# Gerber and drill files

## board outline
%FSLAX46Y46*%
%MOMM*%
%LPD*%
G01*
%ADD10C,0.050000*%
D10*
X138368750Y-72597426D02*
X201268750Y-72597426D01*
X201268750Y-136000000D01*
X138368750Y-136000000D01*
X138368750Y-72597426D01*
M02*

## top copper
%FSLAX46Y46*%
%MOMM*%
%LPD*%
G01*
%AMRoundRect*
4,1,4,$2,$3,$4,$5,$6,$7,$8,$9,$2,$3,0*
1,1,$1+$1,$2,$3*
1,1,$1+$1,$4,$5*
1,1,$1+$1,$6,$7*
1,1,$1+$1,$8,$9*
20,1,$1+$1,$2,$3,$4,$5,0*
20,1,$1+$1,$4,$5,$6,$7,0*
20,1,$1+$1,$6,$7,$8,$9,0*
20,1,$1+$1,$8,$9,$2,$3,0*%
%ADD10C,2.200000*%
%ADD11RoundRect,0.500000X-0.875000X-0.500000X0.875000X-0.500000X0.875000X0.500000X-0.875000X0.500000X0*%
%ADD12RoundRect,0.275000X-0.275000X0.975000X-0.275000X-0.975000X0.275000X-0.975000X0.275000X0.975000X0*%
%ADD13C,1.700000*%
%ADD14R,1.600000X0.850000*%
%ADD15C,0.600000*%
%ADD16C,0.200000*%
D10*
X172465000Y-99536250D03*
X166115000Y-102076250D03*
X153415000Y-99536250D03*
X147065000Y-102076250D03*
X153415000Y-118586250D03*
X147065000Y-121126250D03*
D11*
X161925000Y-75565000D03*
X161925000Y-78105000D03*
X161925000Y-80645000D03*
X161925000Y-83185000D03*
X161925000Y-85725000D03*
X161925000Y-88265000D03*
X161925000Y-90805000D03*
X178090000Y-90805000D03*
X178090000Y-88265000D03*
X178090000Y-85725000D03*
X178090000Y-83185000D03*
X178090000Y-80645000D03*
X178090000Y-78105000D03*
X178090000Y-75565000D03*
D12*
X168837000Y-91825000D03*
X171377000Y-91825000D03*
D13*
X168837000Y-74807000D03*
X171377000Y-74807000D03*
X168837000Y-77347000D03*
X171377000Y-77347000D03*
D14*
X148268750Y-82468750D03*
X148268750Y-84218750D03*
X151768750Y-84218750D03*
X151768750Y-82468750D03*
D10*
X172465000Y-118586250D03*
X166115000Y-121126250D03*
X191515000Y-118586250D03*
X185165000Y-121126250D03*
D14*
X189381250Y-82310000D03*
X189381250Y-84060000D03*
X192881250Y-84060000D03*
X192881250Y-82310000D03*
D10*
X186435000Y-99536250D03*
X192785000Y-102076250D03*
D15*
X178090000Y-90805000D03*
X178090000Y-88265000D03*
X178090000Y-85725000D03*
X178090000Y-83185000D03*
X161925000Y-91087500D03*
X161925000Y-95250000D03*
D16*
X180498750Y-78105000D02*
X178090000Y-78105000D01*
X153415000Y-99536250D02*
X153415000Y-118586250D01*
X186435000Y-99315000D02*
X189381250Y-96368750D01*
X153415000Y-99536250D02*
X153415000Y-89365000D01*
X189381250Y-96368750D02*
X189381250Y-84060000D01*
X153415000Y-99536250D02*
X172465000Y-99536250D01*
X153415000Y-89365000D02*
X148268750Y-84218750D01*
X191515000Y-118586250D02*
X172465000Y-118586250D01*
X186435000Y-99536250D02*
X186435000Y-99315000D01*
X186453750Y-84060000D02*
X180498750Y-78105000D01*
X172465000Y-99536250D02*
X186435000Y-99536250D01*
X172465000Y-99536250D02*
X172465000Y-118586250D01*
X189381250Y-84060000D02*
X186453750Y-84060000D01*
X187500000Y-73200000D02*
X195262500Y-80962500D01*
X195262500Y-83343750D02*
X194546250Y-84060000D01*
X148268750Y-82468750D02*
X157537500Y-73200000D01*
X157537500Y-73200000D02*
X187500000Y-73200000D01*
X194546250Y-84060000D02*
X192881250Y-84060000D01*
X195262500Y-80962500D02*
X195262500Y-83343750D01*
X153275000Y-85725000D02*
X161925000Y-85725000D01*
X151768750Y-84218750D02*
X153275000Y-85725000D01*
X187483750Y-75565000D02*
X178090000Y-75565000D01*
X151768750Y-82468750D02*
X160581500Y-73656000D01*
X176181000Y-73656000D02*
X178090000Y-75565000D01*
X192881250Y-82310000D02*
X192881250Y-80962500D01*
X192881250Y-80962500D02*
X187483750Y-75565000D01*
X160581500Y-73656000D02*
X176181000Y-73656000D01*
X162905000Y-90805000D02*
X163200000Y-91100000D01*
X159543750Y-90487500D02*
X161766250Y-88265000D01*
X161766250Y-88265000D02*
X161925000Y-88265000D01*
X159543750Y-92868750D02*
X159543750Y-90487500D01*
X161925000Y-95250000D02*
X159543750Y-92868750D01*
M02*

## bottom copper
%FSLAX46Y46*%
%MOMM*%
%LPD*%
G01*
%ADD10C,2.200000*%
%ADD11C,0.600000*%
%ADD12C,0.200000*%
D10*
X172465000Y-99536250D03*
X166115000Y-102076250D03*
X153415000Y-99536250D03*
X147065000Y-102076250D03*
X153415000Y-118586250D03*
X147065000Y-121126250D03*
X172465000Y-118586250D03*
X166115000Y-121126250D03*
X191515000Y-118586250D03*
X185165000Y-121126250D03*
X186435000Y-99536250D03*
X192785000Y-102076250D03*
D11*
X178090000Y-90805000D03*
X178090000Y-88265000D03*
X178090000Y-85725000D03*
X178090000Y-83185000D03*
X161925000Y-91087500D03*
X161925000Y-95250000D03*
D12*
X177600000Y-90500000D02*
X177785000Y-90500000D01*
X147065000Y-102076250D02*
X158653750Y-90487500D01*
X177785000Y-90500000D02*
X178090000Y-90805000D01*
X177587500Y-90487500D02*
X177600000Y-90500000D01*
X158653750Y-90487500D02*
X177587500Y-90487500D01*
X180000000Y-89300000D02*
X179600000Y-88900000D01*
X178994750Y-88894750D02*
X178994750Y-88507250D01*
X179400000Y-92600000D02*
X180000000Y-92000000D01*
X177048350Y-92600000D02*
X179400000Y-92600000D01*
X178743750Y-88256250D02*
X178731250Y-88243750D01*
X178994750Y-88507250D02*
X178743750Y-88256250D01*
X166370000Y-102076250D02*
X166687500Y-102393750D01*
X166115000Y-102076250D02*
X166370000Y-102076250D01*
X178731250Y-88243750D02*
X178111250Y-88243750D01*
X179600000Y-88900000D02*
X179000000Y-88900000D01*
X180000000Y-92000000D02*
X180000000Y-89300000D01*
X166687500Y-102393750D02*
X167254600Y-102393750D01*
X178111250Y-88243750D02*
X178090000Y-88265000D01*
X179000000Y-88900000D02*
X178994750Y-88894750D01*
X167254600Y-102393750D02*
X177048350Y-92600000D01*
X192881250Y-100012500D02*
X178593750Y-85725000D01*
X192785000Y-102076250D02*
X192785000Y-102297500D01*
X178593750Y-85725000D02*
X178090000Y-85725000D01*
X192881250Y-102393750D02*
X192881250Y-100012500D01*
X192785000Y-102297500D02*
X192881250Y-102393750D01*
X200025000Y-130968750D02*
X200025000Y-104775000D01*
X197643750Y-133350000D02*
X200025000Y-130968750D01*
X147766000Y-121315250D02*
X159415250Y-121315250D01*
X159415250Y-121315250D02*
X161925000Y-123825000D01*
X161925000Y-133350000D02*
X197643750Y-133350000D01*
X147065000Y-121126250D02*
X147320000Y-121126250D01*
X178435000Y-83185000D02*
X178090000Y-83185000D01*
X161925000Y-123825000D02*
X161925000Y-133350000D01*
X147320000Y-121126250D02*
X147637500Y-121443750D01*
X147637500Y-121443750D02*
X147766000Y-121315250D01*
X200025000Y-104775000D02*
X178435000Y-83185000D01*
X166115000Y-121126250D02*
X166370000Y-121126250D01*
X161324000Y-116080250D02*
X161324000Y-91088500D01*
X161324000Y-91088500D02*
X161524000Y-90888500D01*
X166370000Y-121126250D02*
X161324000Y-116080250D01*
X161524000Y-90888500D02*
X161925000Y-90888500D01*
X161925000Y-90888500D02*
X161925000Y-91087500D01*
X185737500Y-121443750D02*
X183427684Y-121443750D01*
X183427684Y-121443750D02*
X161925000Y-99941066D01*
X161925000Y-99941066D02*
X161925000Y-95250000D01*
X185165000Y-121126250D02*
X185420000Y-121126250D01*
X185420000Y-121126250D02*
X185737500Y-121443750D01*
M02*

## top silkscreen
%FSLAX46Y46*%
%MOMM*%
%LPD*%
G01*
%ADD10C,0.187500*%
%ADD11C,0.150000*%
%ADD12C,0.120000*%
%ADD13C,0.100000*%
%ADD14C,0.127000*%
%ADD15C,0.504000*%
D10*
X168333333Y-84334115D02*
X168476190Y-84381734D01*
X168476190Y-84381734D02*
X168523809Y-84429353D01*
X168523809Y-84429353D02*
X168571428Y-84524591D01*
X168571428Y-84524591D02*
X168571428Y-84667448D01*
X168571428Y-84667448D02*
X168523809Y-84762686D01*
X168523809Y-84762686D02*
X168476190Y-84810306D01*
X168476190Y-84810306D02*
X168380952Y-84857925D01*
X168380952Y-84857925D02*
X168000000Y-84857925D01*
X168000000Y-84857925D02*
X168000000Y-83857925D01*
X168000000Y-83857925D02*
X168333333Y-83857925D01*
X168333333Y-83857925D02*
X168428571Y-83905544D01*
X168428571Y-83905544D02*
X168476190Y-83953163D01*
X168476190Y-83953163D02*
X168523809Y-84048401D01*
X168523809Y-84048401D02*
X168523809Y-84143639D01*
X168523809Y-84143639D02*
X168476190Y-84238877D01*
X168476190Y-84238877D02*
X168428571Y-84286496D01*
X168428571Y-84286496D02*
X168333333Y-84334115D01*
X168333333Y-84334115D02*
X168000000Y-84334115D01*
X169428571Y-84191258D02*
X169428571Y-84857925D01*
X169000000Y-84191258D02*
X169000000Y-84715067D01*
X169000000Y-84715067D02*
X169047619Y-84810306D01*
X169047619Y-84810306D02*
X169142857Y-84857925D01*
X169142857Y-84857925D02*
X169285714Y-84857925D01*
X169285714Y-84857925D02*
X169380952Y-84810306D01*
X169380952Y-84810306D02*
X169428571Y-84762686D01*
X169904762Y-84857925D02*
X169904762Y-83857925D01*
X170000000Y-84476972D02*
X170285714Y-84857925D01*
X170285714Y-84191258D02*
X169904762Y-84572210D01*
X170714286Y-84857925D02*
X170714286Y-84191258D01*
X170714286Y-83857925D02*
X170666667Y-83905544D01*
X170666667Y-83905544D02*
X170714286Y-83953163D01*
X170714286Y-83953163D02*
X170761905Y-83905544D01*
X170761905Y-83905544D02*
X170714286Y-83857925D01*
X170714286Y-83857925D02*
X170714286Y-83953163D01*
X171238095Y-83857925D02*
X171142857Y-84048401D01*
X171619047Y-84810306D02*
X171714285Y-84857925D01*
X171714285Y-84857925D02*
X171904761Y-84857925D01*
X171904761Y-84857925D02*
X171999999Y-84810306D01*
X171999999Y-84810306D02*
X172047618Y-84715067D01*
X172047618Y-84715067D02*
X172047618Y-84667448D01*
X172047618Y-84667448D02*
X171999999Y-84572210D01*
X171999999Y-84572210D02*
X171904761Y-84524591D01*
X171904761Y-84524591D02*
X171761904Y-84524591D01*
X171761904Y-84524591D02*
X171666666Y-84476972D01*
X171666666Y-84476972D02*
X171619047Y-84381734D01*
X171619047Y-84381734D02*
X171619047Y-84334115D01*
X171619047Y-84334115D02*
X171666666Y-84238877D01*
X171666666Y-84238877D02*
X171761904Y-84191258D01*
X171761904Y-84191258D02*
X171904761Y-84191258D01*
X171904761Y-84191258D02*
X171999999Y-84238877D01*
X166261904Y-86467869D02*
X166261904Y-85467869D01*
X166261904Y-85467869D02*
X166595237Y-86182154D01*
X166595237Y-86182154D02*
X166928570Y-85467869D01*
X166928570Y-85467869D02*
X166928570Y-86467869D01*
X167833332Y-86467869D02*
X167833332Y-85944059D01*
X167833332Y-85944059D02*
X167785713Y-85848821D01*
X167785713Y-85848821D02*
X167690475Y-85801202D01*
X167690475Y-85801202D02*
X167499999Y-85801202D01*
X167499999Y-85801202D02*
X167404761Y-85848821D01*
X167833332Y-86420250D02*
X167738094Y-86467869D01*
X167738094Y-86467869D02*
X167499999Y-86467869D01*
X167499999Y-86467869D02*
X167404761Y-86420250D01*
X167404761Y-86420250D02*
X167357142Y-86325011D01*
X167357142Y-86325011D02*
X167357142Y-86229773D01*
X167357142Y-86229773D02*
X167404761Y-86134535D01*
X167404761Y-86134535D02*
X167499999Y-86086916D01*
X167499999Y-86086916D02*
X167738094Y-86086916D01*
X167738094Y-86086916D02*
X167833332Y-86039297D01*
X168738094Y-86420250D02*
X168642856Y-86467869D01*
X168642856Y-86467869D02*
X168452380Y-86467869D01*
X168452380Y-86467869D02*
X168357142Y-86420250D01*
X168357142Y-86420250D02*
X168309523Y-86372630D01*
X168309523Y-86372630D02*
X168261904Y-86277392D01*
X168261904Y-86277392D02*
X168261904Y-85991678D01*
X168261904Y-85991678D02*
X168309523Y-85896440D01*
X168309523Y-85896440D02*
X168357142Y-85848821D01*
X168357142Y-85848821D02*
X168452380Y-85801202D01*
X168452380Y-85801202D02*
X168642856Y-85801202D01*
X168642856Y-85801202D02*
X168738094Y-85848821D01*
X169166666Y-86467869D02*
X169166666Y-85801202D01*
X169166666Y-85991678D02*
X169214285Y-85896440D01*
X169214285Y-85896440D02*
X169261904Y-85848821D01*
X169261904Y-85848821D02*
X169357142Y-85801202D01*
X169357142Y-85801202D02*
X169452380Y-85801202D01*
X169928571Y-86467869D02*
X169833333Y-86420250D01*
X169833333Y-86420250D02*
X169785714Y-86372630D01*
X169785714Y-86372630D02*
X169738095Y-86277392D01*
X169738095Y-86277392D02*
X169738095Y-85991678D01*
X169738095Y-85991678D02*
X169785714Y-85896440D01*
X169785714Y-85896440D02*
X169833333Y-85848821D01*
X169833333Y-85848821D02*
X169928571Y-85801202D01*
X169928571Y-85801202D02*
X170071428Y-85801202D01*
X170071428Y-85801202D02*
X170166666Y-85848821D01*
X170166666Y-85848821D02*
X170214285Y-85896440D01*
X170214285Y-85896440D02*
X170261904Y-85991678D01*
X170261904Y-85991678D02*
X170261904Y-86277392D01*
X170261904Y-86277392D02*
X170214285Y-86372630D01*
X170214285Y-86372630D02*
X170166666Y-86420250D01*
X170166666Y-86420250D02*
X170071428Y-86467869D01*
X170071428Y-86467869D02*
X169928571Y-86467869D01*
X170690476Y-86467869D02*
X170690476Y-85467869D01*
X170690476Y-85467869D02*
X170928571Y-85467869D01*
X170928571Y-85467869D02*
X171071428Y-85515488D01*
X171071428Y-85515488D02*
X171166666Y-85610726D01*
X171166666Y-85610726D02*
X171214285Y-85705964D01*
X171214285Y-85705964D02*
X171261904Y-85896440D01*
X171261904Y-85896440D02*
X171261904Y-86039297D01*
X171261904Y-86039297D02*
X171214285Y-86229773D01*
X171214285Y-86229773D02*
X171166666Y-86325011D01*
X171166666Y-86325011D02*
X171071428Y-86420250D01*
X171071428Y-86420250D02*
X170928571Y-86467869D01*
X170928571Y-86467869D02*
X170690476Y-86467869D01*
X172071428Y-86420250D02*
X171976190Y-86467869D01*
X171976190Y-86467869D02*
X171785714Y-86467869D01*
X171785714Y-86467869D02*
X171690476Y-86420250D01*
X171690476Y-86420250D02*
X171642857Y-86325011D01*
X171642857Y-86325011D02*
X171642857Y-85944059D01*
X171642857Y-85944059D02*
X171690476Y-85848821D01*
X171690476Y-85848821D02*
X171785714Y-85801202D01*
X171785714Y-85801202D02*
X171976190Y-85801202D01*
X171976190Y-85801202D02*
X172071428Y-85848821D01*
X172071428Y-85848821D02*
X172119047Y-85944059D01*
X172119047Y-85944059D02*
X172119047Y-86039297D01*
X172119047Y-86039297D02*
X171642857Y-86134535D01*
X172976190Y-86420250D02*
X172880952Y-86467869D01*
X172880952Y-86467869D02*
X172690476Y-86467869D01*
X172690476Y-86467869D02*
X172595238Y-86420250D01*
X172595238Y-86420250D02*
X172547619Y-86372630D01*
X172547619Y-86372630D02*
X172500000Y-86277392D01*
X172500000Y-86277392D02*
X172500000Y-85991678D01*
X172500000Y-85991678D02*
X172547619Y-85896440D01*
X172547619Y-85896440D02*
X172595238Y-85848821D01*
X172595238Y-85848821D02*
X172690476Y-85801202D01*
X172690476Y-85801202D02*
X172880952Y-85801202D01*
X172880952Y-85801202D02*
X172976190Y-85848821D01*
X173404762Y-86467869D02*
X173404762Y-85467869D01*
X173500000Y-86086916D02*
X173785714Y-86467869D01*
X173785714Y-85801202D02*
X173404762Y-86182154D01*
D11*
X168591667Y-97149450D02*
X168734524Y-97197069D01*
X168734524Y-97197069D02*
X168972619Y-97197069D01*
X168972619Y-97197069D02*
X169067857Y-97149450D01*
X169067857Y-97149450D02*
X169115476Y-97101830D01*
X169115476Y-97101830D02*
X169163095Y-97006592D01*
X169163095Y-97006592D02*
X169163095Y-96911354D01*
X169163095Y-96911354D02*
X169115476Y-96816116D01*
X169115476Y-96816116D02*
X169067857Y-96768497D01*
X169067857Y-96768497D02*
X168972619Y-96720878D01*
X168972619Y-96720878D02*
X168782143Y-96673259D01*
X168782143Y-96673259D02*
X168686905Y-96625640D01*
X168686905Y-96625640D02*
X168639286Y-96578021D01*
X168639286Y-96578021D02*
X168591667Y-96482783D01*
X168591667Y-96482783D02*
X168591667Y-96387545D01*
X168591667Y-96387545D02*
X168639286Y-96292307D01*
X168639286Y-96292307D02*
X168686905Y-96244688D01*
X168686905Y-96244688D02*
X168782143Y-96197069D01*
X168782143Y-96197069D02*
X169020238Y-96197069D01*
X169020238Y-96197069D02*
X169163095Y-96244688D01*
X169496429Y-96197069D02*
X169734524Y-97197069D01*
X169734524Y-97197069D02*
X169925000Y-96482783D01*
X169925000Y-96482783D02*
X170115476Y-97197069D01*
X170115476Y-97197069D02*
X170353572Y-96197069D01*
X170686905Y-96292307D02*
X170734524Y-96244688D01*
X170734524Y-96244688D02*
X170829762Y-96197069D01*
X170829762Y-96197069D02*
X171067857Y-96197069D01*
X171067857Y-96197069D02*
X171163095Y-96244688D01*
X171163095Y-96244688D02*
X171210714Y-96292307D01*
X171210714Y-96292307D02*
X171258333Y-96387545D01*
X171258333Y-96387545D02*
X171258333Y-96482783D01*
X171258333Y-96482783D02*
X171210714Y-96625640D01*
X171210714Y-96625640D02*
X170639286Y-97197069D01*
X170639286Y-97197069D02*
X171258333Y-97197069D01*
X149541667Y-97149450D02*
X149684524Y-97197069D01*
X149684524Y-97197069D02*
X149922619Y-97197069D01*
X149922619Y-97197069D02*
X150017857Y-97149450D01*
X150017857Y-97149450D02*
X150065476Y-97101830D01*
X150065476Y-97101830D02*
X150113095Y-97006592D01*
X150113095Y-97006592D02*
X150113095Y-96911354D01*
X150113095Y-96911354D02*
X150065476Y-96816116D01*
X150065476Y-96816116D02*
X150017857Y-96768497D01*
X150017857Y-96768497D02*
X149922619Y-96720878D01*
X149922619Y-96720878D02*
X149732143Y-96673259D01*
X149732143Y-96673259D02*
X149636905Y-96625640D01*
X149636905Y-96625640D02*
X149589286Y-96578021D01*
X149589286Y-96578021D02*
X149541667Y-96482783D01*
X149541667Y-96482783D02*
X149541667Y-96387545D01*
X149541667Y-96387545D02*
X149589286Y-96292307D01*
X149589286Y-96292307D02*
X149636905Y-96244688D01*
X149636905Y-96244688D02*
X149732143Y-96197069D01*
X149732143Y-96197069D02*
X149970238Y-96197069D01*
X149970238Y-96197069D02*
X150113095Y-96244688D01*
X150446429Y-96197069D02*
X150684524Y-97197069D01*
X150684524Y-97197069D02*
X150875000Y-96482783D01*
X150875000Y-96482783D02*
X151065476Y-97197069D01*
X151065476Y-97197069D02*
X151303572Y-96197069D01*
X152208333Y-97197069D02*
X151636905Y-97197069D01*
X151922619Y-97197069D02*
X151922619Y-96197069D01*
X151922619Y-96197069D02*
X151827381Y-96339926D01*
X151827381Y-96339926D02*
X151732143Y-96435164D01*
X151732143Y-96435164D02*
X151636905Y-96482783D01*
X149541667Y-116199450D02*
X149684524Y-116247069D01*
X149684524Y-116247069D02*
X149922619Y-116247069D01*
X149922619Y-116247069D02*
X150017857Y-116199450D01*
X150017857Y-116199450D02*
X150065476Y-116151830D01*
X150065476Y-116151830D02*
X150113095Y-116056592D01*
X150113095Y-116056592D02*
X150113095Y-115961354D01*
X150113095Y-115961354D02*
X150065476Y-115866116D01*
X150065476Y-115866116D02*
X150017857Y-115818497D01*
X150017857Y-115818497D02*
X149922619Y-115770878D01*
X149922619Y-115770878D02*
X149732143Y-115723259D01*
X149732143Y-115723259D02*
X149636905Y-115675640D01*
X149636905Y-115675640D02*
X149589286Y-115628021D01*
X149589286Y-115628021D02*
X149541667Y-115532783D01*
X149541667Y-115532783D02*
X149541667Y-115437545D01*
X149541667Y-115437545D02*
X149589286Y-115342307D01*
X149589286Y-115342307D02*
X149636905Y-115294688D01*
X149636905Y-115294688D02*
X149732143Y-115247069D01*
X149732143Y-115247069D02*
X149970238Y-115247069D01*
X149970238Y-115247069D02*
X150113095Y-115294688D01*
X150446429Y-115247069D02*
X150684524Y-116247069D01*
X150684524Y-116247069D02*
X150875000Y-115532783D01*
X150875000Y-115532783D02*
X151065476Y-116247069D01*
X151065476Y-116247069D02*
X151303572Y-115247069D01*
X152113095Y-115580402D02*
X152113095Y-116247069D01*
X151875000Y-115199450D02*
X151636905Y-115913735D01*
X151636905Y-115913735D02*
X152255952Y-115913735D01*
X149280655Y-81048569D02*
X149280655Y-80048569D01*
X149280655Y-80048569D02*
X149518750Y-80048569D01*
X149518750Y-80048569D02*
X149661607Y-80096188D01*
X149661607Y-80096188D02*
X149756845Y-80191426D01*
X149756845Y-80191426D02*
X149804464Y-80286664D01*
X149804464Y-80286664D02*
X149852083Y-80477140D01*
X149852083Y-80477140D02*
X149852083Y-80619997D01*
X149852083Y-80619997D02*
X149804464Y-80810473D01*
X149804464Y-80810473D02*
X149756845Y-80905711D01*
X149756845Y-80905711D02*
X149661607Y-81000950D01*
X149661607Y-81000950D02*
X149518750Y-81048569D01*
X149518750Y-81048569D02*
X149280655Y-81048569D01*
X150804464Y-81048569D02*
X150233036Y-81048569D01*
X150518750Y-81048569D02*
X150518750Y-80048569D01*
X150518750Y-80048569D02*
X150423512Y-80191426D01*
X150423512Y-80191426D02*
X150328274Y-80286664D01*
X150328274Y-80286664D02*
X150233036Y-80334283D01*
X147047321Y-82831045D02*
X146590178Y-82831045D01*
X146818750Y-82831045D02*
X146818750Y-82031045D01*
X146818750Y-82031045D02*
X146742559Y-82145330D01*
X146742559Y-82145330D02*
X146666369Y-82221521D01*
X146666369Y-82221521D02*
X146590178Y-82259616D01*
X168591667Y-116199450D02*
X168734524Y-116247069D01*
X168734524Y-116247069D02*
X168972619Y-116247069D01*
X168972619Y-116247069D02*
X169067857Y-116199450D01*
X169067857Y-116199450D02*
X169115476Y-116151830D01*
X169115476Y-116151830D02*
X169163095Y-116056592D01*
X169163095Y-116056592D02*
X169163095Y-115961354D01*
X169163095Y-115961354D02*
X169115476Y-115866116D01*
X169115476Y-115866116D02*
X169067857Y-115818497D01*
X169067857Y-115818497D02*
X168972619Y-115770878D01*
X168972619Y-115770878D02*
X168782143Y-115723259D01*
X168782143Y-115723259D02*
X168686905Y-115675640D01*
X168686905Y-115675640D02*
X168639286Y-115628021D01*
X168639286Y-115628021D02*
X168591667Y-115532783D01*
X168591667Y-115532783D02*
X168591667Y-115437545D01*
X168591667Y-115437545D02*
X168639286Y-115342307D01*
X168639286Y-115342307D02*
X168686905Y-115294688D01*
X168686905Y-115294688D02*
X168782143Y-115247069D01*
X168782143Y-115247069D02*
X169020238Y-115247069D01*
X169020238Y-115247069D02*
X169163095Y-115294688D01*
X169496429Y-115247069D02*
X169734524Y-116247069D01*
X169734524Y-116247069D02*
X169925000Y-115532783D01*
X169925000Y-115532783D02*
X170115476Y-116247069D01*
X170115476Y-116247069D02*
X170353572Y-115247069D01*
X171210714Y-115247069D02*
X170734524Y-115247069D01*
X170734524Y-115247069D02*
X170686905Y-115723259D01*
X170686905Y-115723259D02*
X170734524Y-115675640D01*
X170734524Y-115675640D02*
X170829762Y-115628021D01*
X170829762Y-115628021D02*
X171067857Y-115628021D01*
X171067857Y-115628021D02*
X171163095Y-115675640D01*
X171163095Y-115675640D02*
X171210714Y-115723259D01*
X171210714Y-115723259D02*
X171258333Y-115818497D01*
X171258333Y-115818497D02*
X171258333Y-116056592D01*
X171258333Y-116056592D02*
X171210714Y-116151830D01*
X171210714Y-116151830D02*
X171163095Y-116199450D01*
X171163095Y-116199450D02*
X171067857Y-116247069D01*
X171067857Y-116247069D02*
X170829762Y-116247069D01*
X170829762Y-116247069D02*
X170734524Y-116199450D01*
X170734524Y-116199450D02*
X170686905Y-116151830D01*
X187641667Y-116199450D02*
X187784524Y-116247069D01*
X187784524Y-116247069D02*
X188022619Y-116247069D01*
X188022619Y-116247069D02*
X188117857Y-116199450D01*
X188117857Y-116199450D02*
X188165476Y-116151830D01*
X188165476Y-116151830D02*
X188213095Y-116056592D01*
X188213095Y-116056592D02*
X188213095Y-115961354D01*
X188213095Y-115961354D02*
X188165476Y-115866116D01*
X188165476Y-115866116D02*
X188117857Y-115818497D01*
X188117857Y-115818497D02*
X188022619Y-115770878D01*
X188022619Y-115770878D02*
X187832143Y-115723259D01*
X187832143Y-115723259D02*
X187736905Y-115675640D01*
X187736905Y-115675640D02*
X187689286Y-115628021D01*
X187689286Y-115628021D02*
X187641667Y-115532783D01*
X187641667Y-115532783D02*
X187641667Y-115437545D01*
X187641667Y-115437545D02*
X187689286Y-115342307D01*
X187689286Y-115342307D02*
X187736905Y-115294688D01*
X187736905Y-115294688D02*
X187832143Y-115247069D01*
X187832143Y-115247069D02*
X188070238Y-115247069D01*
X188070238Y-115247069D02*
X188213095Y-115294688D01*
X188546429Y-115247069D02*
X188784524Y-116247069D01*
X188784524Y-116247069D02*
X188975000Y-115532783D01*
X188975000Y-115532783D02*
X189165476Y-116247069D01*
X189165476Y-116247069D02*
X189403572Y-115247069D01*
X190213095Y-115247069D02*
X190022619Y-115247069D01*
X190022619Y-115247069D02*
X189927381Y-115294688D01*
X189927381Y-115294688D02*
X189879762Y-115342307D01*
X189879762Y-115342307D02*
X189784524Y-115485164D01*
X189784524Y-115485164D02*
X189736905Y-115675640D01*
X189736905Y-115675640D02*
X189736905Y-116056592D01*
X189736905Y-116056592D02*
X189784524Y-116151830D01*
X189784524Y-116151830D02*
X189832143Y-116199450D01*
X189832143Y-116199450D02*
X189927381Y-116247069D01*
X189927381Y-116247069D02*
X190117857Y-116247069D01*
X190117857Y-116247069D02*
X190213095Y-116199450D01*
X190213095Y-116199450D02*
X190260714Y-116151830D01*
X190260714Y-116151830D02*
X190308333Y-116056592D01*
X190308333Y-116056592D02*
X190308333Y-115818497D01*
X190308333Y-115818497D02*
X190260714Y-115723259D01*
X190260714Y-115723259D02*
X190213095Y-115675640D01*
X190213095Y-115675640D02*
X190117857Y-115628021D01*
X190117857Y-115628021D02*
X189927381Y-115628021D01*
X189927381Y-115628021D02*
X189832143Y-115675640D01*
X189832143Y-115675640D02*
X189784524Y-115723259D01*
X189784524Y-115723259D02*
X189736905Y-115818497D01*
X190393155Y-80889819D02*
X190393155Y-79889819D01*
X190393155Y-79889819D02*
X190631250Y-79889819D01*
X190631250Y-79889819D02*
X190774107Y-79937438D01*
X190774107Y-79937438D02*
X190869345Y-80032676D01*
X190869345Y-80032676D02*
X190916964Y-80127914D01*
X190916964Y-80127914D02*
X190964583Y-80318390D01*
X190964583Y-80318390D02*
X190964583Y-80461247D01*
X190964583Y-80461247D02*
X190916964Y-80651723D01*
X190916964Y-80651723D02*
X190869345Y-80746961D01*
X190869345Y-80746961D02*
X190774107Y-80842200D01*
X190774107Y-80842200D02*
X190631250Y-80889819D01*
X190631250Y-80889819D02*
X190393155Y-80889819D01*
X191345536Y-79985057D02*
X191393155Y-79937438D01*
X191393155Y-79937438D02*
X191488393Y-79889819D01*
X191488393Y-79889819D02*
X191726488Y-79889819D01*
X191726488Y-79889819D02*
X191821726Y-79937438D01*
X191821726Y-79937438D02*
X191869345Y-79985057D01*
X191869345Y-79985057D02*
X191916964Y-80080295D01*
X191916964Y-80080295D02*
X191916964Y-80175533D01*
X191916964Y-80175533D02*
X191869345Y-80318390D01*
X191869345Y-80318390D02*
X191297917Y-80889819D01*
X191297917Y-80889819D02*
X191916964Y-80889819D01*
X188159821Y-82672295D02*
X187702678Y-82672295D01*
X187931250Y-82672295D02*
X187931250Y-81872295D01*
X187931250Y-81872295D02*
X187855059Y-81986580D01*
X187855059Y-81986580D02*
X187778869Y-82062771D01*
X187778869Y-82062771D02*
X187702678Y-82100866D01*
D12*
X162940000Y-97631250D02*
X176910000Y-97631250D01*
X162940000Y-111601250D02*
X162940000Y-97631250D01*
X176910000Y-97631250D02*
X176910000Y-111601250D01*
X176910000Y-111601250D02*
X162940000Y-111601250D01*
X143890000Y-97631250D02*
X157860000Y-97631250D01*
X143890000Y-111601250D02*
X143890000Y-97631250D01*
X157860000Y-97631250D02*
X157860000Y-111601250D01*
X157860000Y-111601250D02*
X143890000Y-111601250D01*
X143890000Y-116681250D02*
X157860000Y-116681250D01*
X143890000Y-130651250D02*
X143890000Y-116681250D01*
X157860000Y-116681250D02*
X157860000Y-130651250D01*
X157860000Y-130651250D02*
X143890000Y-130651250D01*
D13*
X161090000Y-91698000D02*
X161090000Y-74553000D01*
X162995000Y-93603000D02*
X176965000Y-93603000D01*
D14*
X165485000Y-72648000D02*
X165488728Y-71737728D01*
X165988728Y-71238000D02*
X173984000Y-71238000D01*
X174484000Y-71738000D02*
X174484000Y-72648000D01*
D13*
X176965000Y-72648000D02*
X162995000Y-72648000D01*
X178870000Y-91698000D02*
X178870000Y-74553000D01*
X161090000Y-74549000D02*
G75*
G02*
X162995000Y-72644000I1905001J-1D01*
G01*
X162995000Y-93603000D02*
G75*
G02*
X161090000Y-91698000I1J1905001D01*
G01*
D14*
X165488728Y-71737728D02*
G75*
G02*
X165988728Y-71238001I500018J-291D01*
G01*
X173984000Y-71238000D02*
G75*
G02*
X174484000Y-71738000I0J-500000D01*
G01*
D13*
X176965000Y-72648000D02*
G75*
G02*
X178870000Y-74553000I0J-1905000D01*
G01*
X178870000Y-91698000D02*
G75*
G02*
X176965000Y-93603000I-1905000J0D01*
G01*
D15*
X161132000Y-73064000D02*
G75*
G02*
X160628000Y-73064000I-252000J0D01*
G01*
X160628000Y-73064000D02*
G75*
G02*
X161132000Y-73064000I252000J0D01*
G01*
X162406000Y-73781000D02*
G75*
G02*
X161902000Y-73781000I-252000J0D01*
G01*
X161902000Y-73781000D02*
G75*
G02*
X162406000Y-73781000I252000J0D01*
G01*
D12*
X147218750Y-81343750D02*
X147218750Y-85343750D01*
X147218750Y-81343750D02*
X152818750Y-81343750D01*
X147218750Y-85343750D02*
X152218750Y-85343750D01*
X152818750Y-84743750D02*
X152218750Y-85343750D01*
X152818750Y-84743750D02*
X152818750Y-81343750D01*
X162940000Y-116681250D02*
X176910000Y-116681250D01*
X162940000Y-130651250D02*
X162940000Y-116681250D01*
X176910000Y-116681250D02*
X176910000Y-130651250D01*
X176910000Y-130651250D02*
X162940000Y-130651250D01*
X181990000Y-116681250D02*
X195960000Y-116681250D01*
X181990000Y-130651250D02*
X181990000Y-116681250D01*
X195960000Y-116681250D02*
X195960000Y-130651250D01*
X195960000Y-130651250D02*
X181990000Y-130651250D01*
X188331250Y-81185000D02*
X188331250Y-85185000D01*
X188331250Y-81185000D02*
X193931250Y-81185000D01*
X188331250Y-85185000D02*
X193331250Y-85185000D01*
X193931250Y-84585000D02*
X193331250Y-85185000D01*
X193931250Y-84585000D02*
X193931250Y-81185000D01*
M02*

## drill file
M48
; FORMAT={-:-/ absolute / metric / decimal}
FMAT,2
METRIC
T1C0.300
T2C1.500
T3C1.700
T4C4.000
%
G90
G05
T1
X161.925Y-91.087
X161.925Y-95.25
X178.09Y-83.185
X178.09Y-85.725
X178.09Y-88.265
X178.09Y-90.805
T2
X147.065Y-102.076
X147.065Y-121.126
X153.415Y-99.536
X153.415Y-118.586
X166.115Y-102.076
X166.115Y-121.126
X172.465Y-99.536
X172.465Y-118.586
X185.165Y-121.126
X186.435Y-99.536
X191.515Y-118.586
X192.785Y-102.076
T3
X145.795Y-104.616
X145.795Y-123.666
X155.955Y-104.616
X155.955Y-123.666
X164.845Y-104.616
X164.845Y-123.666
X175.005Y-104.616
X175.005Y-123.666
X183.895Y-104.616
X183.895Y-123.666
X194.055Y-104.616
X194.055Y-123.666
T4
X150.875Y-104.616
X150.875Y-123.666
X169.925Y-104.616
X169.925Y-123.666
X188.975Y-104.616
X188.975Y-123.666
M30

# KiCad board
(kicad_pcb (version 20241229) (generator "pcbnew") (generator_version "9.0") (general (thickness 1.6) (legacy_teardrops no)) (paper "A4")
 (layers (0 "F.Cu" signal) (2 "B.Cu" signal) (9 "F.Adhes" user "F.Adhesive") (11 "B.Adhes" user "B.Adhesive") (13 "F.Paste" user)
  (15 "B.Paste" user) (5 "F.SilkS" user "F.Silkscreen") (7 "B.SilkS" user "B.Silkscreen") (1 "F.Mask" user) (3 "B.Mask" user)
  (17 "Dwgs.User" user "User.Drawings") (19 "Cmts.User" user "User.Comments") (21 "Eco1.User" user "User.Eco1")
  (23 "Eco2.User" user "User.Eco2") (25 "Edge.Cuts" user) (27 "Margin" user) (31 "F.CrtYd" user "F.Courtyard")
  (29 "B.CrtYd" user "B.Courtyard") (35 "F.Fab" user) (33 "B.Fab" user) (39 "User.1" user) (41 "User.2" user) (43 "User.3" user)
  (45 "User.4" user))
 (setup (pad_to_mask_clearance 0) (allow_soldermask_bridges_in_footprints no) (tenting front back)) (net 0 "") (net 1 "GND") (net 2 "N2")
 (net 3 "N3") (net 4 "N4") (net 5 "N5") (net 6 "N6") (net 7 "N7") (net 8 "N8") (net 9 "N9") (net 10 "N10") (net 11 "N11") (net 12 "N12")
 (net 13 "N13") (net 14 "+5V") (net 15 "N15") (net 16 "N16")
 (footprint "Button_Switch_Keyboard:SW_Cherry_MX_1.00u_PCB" (layer "F.Cu") (at 172.465 99.53625)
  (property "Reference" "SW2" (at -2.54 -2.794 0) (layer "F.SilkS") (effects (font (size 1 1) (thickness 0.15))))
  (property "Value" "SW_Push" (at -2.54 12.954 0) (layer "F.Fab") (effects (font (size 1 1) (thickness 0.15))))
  (fp_line (start -9.525 -1.905) (end 4.445 -1.905) (stroke (width 0.12) (type solid)) (layer "F.SilkS"))
  (fp_line (start -9.525 12.065) (end -9.525 -1.905) (stroke (width 0.12) (type solid)) (layer "F.SilkS"))
  (fp_line (start 4.445 -1.905) (end 4.445 12.065) (stroke (width 0.12) (type solid)) (layer "F.SilkS"))
  (fp_line (start 4.445 12.065) (end -9.525 12.065) (stroke (width 0.12) (type solid)) (layer "F.SilkS"))
  (pad "" np_thru_hole circle (at -7.62 5.08) (size 1.7 1.7) (drill 1.7) (layers "*.Cu" "*.Mask"))
  (pad "" np_thru_hole circle (at -2.54 5.08) (size 4 4) (drill 4) (layers "*.Cu" "*.Mask"))
  (pad "" np_thru_hole circle (at 2.54 5.08) (size 1.7 1.7) (drill 1.7) (layers "*.Cu" "*.Mask"))
  (pad "1" thru_hole circle (at 0 0) (size 2.2 2.2) (drill 1.5) (layers "*.Cu" "*.Mask") (remove_unused_layers no) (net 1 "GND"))
  (pad "2" thru_hole circle (at -6.35 2.54) (size 2.2 2.2) (drill 1.5) (layers "*.Cu" "*.Mask") (remove_unused_layers no) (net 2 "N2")))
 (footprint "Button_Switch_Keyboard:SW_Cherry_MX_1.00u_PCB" (layer "F.Cu") (at 153.415 99.53625)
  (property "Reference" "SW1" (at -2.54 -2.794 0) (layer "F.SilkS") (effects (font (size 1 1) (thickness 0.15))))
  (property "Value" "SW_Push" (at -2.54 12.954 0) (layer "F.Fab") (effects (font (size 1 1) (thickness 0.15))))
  (fp_line (start -9.525 -1.905) (end 4.445 -1.905) (stroke (width 0.12) (type solid)) (layer "F.SilkS"))
  (fp_line (start -9.525 12.065) (end -9.525 -1.905) (stroke (width 0.12) (type solid)) (layer "F.SilkS"))
  (fp_line (start 4.445 -1.905) (end 4.445 12.065) (stroke (width 0.12) (type solid)) (layer "F.SilkS"))
  (fp_line (start 4.445 12.065) (end -9.525 12.065) (stroke (width 0.12) (type solid)) (layer "F.SilkS"))
  (pad "" np_thru_hole circle (at -7.62 5.08) (size 1.7 1.7) (drill 1.7) (layers "*.Cu" "*.Mask"))
  (pad "" np_thru_hole circle (at -2.54 5.08) (size 4 4) (drill 4) (layers "*.Cu" "*.Mask"))
  (pad "" np_thru_hole circle (at 2.54 5.08) (size 1.7 1.7) (drill 1.7) (layers "*.Cu" "*.Mask"))
  (pad "1" thru_hole circle (at 0 0) (size 2.2 2.2) (drill 1.5) (layers "*.Cu" "*.Mask") (remove_unused_layers no) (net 1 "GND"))
  (pad "2" thru_hole circle (at -6.35 2.54) (size 2.2 2.2) (drill 1.5) (layers "*.Cu" "*.Mask") (remove_unused_layers no) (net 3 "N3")))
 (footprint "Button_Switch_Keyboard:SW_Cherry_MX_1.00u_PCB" (layer "F.Cu") (at 153.415 118.58625)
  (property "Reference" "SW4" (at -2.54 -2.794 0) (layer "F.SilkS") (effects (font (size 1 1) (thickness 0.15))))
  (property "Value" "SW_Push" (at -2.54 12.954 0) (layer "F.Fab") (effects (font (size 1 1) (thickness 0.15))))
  (fp_line (start -9.525 -1.905) (end 4.445 -1.905) (stroke (width 0.12) (type solid)) (layer "F.SilkS"))
  (fp_line (start -9.525 12.065) (end -9.525 -1.905) (stroke (width 0.12) (type solid)) (layer "F.SilkS"))
  (fp_line (start 4.445 -1.905) (end 4.445 12.065) (stroke (width 0.12) (type solid)) (layer "F.SilkS"))
  (fp_line (start 4.445 12.065) (end -9.525 12.065) (stroke (width 0.12) (type solid)) (layer "F.SilkS"))
  (pad "" np_thru_hole circle (at -7.62 5.08) (size 1.7 1.7) (drill 1.7) (layers "*.Cu" "*.Mask"))
  (pad "" np_thru_hole circle (at -2.54 5.08) (size 4 4) (drill 4) (layers "*.Cu" "*.Mask"))
  (pad "" np_thru_hole circle (at 2.54 5.08) (size 1.7 1.7) (drill 1.7) (layers "*.Cu" "*.Mask"))
  (pad "1" thru_hole circle (at 0 0) (size 2.2 2.2) (drill 1.5) (layers "*.Cu" "*.Mask") (remove_unused_layers no) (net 1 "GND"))
  (pad "2" thru_hole circle (at -6.35 2.54) (size 2.2 2.2) (drill 1.5) (layers "*.Cu" "*.Mask") (remove_unused_layers no) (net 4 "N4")))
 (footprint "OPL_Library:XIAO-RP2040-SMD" (layer "F.Cu") (at 169.925 83.185)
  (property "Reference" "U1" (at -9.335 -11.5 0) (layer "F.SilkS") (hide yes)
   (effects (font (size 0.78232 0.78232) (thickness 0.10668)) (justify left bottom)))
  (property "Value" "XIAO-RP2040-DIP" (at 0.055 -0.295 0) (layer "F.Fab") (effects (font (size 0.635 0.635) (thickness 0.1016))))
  (fp_line (start -8.835 8.513) (end -8.835 -8.632) (stroke (width 0.1) (type solid)) (layer "F.SilkS"))
  (fp_line (start -6.93 10.418) (end 7.04 10.418) (stroke (width 0.1) (type solid)) (layer "F.SilkS"))
  (fp_line (start -4.44 -10.537) (end -4.436272 -11.447272) (stroke (width 0.127) (type solid)) (layer "F.SilkS"))
  (fp_line (start -3.936272 -11.947) (end 4.059 -11.947) (stroke (width 0.127) (type solid)) (layer "F.SilkS"))
  (fp_line (start 4.559 -11.447) (end 4.559 -10.537) (stroke (width 0.127) (type solid)) (layer "F.SilkS"))
  (fp_line (start 7.04 -10.537) (end -6.93 -10.537) (stroke (width 0.1) (type solid)) (layer "F.SilkS"))
  (fp_line (start 8.945 8.513) (end 8.945 -8.632) (stroke (width 0.1) (type solid)) (layer "F.SilkS"))
  (fp_arc (start -8.835 -8.636) (mid -8.277038 -9.983038) (end -6.93 -10.541) (stroke (width 0.1) (type solid)) (layer "F.SilkS"))
  (fp_arc (start -6.93 10.418) (mid -8.277038 9.860038) (end -8.835 8.513) (stroke (width 0.1) (type solid)) (layer "F.SilkS"))
  (fp_arc (start -4.436272 -11.447272) (mid -4.289724 -11.800644) (end -3.936272 -11.947) (stroke (width 0.127) (type default))
   (layer "F.SilkS"))
  (fp_arc (start 4.059 -11.947) (mid 4.412553 -11.800553) (end 4.559 -11.447) (stroke (width 0.127) (type default)) (layer "F.SilkS"))
  (fp_arc (start 7.04 -10.537) (mid 8.387038 -9.979038) (end 8.945 -8.632) (stroke (width 0.1) (type solid)) (layer "F.SilkS"))
  (fp_arc (start 8.945 8.513) (mid 8.387038 9.860038) (end 7.04 10.418) (stroke (width 0.1) (type solid)) (layer "F.SilkS"))
  (fp_circle (center -9.045 -10.121) (end -9.045 -10.375) (stroke (width 0.5) (type solid)) (fill yes) (layer "F.SilkS"))
  (fp_circle (center -7.771 -9.404) (end -7.771 -9.658) (stroke (width 0.5) (type solid)) (fill yes) (layer "F.SilkS"))
  (pad "1" smd roundrect (at -8 -7.62) (size 2.75 2) (layers "F.Cu" "F.Mask" "F.Paste") (roundrect_rratio 0.25) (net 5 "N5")
   (solder_mask_margin 0.0508) (thermal_bridge_angle 45))
  (pad "2" smd roundrect (at -8 -5.08) (size 2.75 2) (layers "F.Cu" "F.Mask" "F.Paste") (roundrect_rratio 0.25) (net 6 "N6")
   (solder_mask_margin 0.0508) (thermal_bridge_angle 45))
  (pad "3" smd roundrect (at -8 -2.54) (size 2.75 2) (layers "F.Cu" "F.Mask" "F.Paste") (roundrect_rratio 0.25) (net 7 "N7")
   (solder_mask_margin 0.0508) (thermal_bridge_angle 45))
  (pad "4" smd roundrect (at -8 0) (size 2.75 2) (layers "F.Cu" "F.Mask" "F.Paste") (roundrect_rratio 0.25) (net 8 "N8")
   (solder_mask_margin 0.0508) (thermal_bridge_angle 45))
  (pad "5" smd roundrect (at -8 2.54) (size 2.75 2) (layers "F.Cu" "F.Mask" "F.Paste") (roundrect_rratio 0.25) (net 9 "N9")
   (solder_mask_margin 0.0508) (thermal_bridge_angle 45))
  (pad "6" smd roundrect (at -8 5.08) (size 2.75 2) (layers "F.Cu" "F.Mask" "F.Paste") (roundrect_rratio 0.25) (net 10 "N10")
   (solder_mask_margin 0.0508) (thermal_bridge_angle 45))
  (pad "7" smd roundrect (at -8 7.62) (size 2.75 2) (layers "F.Cu" "F.Mask" "F.Paste") (roundrect_rratio 0.25) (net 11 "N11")
   (solder_mask_margin 0.0508) (thermal_bridge_angle 45))
  (pad "8" smd roundrect (at 8.165 7.62) (size 2.75 2) (layers "F.Cu" "F.Mask" "F.Paste") (roundrect_rratio 0.25) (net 3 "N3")
   (solder_mask_margin 0.0508) (thermal_bridge_angle 45))
  (pad "9" smd roundrect (at 8.165 5.08) (size 2.75 2) (layers "F.Cu" "F.Mask" "F.Paste") (roundrect_rratio 0.25) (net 2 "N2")
   (solder_mask_margin 0.0508) (thermal_bridge_angle 45))
  (pad "10" smd roundrect (at 8.165 2.54) (size 2.75 2) (layers "F.Cu" "F.Mask" "F.Paste") (roundrect_rratio 0.25) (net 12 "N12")
   (solder_mask_margin 0.0508) (thermal_bridge_angle 45))
  (pad "11" smd roundrect (at 8.165 0) (size 2.75 2) (layers "F.Cu" "F.Mask" "F.Paste") (roundrect_rratio 0.25) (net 4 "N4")
   (solder_mask_margin 0.0508) (thermal_bridge_angle 45))
  (pad "12" smd roundrect (at 8.165 -2.54) (size 2.75 2) (layers "F.Cu" "F.Mask" "F.Paste") (roundrect_rratio 0.25) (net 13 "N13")
   (solder_mask_margin 0.0508) (thermal_bridge_angle 45))
  (pad "13" smd roundrect (at 8.165 -5.08) (size 2.75 2) (layers "F.Cu" "F.Mask" "F.Paste") (roundrect_rratio 0.25) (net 1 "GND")
   (solder_mask_margin 0.0508) (thermal_bridge_angle 45))
  (pad "14" smd roundrect (at 8.165 -7.62) (size 2.75 2) (layers "F.Cu" "F.Mask" "F.Paste") (roundrect_rratio 0.25) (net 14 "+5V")
   (solder_mask_margin 0.0508) (thermal_bridge_angle 45))
  (pad "15" smd roundrect (at -1.088 8.64 270) (size 2.5 1.1) (layers "F.Cu" "F.Mask" "F.Paste") (roundrect_rratio 0.25)
   (thermal_bridge_angle 45))
  (pad "16" smd roundrect (at 1.452 8.64 270) (size 2.5 1.1) (layers "F.Cu" "F.Mask" "F.Paste") (roundrect_rratio 0.25)
   (thermal_bridge_angle 45))
  (pad "17" smd circle (at -1.088 -8.378) (size 1.7 1.7) (layers "F.Cu" "F.Mask" "F.Paste"))
  (pad "18" smd circle (at 1.452 -8.378) (size 1.7 1.7) (layers "F.Cu" "F.Mask" "F.Paste"))
  (pad "19" smd circle (at -1.088 -5.838) (size 1.7 1.7) (layers "F.Cu" "F.Mask" "F.Paste"))
  (pad "20" smd circle (at 1.452 -5.838) (size 1.7 1.7) (layers "F.Cu" "F.Mask" "F.Paste")))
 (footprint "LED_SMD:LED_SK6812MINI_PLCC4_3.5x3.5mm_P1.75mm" (layer "F.Cu") (at 150.01875 83.34375)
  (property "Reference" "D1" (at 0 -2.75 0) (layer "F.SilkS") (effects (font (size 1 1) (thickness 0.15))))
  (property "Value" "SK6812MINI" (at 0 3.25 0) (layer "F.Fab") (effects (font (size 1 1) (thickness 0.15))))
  (fp_line (start -2.8 -2) (end -2.8 2) (stroke (width 0.12) (type default)) (layer "F.SilkS"))
  (fp_line (start -2.8 -2) (end 2.8 -2) (stroke (width 0.12) (type solid)) (layer "F.SilkS"))
  (fp_line (start -2.8 2) (end 2.2 2) (stroke (width 0.12) (type solid)) (layer "F.SilkS"))
  (fp_line (start 2.8 1.4) (end 2.2 2) (stroke (width 0.12) (type default)) (layer "F.SilkS"))
  (fp_line (start 2.8 1.4) (end 2.8 -2) (stroke (width 0.12) (type solid)) (layer "F.SilkS"))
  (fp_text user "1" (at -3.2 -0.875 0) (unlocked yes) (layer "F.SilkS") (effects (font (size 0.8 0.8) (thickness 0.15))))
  (pad "1" smd rect (at -1.75 -0.875) (size 1.6 0.85) (layers "F.Cu" "F.Mask" "F.Paste") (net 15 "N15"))
  (pad "2" smd rect (at -1.75 0.875) (size 1.6 0.85) (layers "F.Cu" "F.Mask" "F.Paste") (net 1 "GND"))
  (pad "3" smd rect (at 1.75 0.875) (size 1.6 0.85) (layers "F.Cu" "F.Mask" "F.Paste") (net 9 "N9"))
  (pad "4" smd rect (at 1.75 -0.875) (size 1.6 0.85) (layers "F.Cu" "F.Mask" "F.Paste") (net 14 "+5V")))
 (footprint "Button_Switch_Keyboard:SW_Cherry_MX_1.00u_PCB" (layer "F.Cu") (at 172.465 118.58625)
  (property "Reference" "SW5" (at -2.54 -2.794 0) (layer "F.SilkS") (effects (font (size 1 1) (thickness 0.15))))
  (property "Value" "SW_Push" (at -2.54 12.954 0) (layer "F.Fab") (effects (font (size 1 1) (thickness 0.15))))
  (fp_line (start -9.525 -1.905) (end 4.445 -1.905) (stroke (width 0.12) (type solid)) (layer "F.SilkS"))
  (fp_line (start -9.525 12.065) (end -9.525 -1.905) (stroke (width 0.12) (type solid)) (layer "F.SilkS"))
  (fp_line (start 4.445 -1.905) (end 4.445 12.065) (stroke (width 0.12) (type solid)) (layer "F.SilkS"))
  (fp_line (start 4.445 12.065) (end -9.525 12.065) (stroke (width 0.12) (type solid)) (layer "F.SilkS"))
  (pad "" np_thru_hole circle (at -7.62 5.08) (size 1.7 1.7) (drill 1.7) (layers "*.Cu" "*.Mask"))
  (pad "" np_thru_hole circle (at -2.54 5.08) (size 4 4) (drill 4) (layers "*.Cu" "*.Mask"))
  (pad "" np_thru_hole circle (at 2.54 5.08) (size 1.7 1.7) (drill 1.7) (layers "*.Cu" "*.Mask"))
  (pad "1" thru_hole circle (at 0 0) (size 2.2 2.2) (drill 1.5) (layers "*.Cu" "*.Mask") (remove_unused_layers no) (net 1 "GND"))
  (pad "2" thru_hole circle (at -6.35 2.54) (size 2.2 2.2) (drill 1.5) (layers "*.Cu" "*.Mask") (remove_unused_layers no) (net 11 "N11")))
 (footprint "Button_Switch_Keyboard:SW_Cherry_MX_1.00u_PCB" (layer "F.Cu") (at 191.515 118.58625)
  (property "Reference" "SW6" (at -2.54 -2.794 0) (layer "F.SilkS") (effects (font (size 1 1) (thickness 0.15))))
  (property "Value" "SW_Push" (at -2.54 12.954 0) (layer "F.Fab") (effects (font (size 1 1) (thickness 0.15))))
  (fp_line (start -9.525 -1.905) (end 4.445 -1.905) (stroke (width 0.12) (type solid)) (layer "F.SilkS"))
  (fp_line (start -9.525 12.065) (end -9.525 -1.905) (stroke (width 0.12) (type solid)) (layer "F.SilkS"))
  (fp_line (start 4.445 -1.905) (end 4.445 12.065) (stroke (width 0.12) (type solid)) (layer "F.SilkS"))
  (fp_line (start 4.445 12.065) (end -9.525 12.065) (stroke (width 0.12) (type solid)) (layer "F.SilkS"))
  (pad "" np_thru_hole circle (at -7.62 5.08) (size 1.7 1.7) (drill 1.7) (layers "*.Cu" "*.Mask"))
  (pad "" np_thru_hole circle (at -2.54 5.08) (size 4 4) (drill 4) (layers "*.Cu" "*.Mask"))
  (pad "" np_thru_hole circle (at 2.54 5.08) (size 1.7 1.7) (drill 1.7) (layers "*.Cu" "*.Mask"))
  (pad "1" thru_hole circle (at 0 0) (size 2.2 2.2) (drill 1.5) (layers "*.Cu" "*.Mask") (remove_unused_layers no) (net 1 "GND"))
  (pad "2" thru_hole circle (at -6.35 2.54) (size 2.2 2.2) (drill 1.5) (layers "*.Cu" "*.Mask") (remove_unused_layers no) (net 10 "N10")))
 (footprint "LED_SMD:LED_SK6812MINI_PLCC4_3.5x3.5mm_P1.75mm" (layer "F.Cu") (at 191.13125 83.185)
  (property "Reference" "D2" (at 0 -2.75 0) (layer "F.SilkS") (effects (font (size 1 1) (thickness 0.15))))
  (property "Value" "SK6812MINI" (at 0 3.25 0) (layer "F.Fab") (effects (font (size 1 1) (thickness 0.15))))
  (fp_line (start -2.8 -2) (end -2.8 2) (stroke (width 0.12) (type default)) (layer "F.SilkS"))
  (fp_line (start -2.8 -2) (end 2.8 -2) (stroke (width 0.12) (type solid)) (layer "F.SilkS"))
  (fp_line (start -2.8 2) (end 2.2 2) (stroke (width 0.12) (type solid)) (layer "F.SilkS"))
  (fp_line (start 2.8 1.4) (end 2.2 2) (stroke (width 0.12) (type default)) (layer "F.SilkS"))
  (fp_line (start 2.8 1.4) (end 2.8 -2) (stroke (width 0.12) (type solid)) (layer "F.SilkS"))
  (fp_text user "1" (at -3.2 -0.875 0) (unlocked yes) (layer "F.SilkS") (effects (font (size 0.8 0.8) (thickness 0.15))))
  (pad "1" smd rect (at -1.75 -0.875) (size 1.6 0.85) (layers "F.Cu" "F.Mask" "F.Paste") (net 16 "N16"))
  (pad "2" smd rect (at -1.75 0.875) (size 1.6 0.85) (layers "F.Cu" "F.Mask" "F.Paste") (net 1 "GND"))
  (pad "3" smd rect (at 1.75 0.875) (size 1.6 0.85) (layers "F.Cu" "F.Mask" "F.Paste") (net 15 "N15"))
  (pad "4" smd rect (at 1.75 -0.875) (size 1.6 0.85) (layers "F.Cu" "F.Mask" "F.Paste") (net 14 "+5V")))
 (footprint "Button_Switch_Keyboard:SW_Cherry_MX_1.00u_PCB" (layer "B.Cu") (at 186.435 99.53625 180)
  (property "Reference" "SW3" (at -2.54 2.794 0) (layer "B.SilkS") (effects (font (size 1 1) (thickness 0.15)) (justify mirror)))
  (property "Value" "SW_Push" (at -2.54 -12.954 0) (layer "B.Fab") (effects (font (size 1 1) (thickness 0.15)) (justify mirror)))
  (pad "" np_thru_hole circle (at -7.62 -5.08 180) (size 1.7 1.7) (drill 1.7) (layers "*.Cu" "*.Mask"))
  (pad "" np_thru_hole circle (at -2.54 -5.08 180) (size 4 4) (drill 4) (layers "*.Cu" "*.Mask"))
  (pad "" np_thru_hole circle (at 2.54 -5.08 180) (size 1.7 1.7) (drill 1.7) (layers "*.Cu" "*.Mask"))
  (pad "1" thru_hole circle (at 0 0 180) (size 2.2 2.2) (drill 1.5) (layers "*.Cu" "*.Mask") (remove_unused_layers no) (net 1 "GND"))
  (pad "2" thru_hole circle (at -6.35 -2.54 180) (size 2.2 2.2) (drill 1.5) (layers "*.Cu" "*.Mask") (remove_unused_layers no)
   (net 12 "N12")))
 (gr_rect (start 138.36875 72.597426) (end 201.26875 136) (stroke (width 0.05) (type default)) (fill no) (layer "Edge.Cuts"))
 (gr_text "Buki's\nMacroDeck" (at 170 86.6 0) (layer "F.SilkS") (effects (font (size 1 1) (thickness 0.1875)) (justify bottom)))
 (segment (start 180.49875 78.105) (end 178.09 78.105) (width 0.2) (layer "F.Cu") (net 1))
 (segment (start 153.415 99.53625) (end 153.415 118.58625) (width 0.2) (layer "F.Cu") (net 1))
 (segment (start 186.435 99.315) (end 189.38125 96.36875) (width 0.2) (layer "F.Cu") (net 1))
 (segment (start 153.415 99.53625) (end 153.415 89.365) (width 0.2) (layer "F.Cu") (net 1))
 (segment (start 189.38125 96.36875) (end 189.38125 84.06) (width 0.2) (layer "F.Cu") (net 1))
 (segment (start 153.415 99.53625) (end 172.465 99.53625) (width 0.2) (layer "F.Cu") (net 1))
 (segment (start 153.415 89.365) (end 148.26875 84.21875) (width 0.2) (layer "F.Cu") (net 1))
 (segment (start 191.515 118.58625) (end 172.465 118.58625) (width 0.2) (layer "F.Cu") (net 1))
 (segment (start 186.435 99.53625) (end 186.435 99.315) (width 0.2) (layer "F.Cu") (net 1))
 (segment (start 186.45375 84.06) (end 180.49875 78.105) (width 0.2) (layer "F.Cu") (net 1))
 (segment (start 172.465 99.53625) (end 186.435 99.53625) (width 0.2) (layer "F.Cu") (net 1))
 (segment (start 172.465 99.53625) (end 172.465 118.58625) (width 0.2) (layer "F.Cu") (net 1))
 (segment (start 189.38125 84.06) (end 186.45375 84.06) (width 0.2) (layer "F.Cu") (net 1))
 (segment (start 187.5 73.2) (end 195.2625 80.9625) (width 0.2) (layer "F.Cu") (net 15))
 (segment (start 195.2625 83.34375) (end 194.54625 84.06) (width 0.2) (layer "F.Cu") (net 15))
 (segment (start 148.26875 82.46875) (end 157.5375 73.2) (width 0.2) (layer "F.Cu") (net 15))
 (segment (start 157.5375 73.2) (end 187.5 73.2) (width 0.2) (layer "F.Cu") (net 15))
 (segment (start 194.54625 84.06) (end 192.88125 84.06) (width 0.2) (layer "F.Cu") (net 15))
 (segment (start 195.2625 80.9625) (end 195.2625 83.34375) (width 0.2) (layer "F.Cu") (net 15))
 (segment (start 153.275 85.725) (end 161.925 85.725) (width 0.2) (layer "F.Cu") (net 9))
 (segment (start 151.76875 84.21875) (end 153.275 85.725) (width 0.2) (layer "F.Cu") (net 9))
 (segment (start 187.48375 75.565) (end 178.09 75.565) (width 0.2) (layer "F.Cu") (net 14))
 (segment (start 151.76875 82.46875) (end 160.5815 73.656) (width 0.2) (layer "F.Cu") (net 14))
 (segment (start 176.181 73.656) (end 178.09 75.565) (width 0.2) (layer "F.Cu") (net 14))
 (segment (start 192.88125 82.31) (end 192.88125 80.9625) (width 0.2) (layer "F.Cu") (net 14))
 (segment (start 192.88125 80.9625) (end 187.48375 75.565) (width 0.2) (layer "F.Cu") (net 14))
 (segment (start 160.5815 73.656) (end 176.181 73.656) (width 0.2) (layer "F.Cu") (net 14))
 (via (at 178.09 90.805) (size 0.6) (drill 0.3) (layers "F.Cu" "B.Cu") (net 3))
 (segment (start 177.6 90.5) (end 177.785 90.5) (width 0.2) (layer "B.Cu") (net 3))
 (segment (start 147.065 102.07625) (end 158.65375 90.4875) (width 0.2) (layer "B.Cu") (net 3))
 (segment (start 177.785 90.5) (end 178.09 90.805) (width 0.2) (layer "B.Cu") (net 3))
 (segment (start 177.5875 90.4875) (end 177.6 90.5) (width 0.2) (layer "B.Cu") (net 3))
 (segment (start 158.65375 90.4875) (end 177.5875 90.4875) (width 0.2) (layer "B.Cu") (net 3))
 (via (at 178.09 88.265) (size 0.6) (drill 0.3) (layers "F.Cu" "B.Cu") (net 2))
 (segment (start 180 89.3) (end 179.6 88.9) (width 0.2) (layer "B.Cu") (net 2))
 (segment (start 178.99475 88.89475) (end 178.99475 88.50725) (width 0.2) (layer "B.Cu") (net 2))
 (segment (start 179.4 92.6) (end 180 92) (width 0.2) (layer "B.Cu") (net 2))
 (segment (start 177.04835 92.6) (end 179.4 92.6) (width 0.2) (layer "B.Cu") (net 2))
 (segment (start 178.74375 88.25625) (end 178.73125 88.24375) (width 0.2) (layer "B.Cu") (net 2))
 (segment (start 178.99475 88.50725) (end 178.74375 88.25625) (width 0.2) (layer "B.Cu") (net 2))
 (segment (start 166.37 102.07625) (end 166.6875 102.39375) (width 0.2) (layer "B.Cu") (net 2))
 (segment (start 166.115 102.07625) (end 166.37 102.07625) (width 0.2) (layer "B.Cu") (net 2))
 (segment (start 178.73125 88.24375) (end 178.11125 88.24375) (width 0.2) (layer "B.Cu") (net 2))
 (segment (start 179.6 88.9) (end 179 88.9) (width 0.2) (layer "B.Cu") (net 2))
 (segment (start 180 92) (end 180 89.3) (width 0.2) (layer "B.Cu") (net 2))
 (segment (start 166.6875 102.39375) (end 167.2546 102.39375) (width 0.2) (layer "B.Cu") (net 2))
 (segment (start 178.11125 88.24375) (end 178.09 88.265) (width 0.2) (layer "B.Cu") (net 2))
 (segment (start 179 88.9) (end 178.99475 88.89475) (width 0.2) (layer "B.Cu") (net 2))
 (segment (start 167.2546 102.39375) (end 177.04835 92.6) (width 0.2) (layer "B.Cu") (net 2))
 (via (at 178.09 85.725) (size 0.6) (drill 0.3) (layers "F.Cu" "B.Cu") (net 12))
 (segment (start 192.88125 100.0125) (end 178.59375 85.725) (width 0.2) (layer "B.Cu") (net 12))
 (segment (start 192.785 102.07625) (end 192.785 102.2975) (width 0.2) (layer "B.Cu") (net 12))
 (segment (start 178.59375 85.725) (end 178.09 85.725) (width 0.2) (layer "B.Cu") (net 12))
 (segment (start 192.88125 102.39375) (end 192.88125 100.0125) (width 0.2) (layer "B.Cu") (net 12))
 (segment (start 192.785 102.2975) (end 192.88125 102.39375) (width 0.2) (layer "B.Cu") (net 12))
 (via (at 178.09 83.185) (size 0.6) (drill 0.3) (layers "F.Cu" "B.Cu") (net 4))
 (segment (start 200.025 130.96875) (end 200.025 104.775) (width 0.2) (layer "B.Cu") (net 4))
 (segment (start 197.64375 133.35) (end 200.025 130.96875) (width 0.2) (layer "B.Cu") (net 4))
 (segment (start 147.766 121.31525) (end 159.41525 121.31525) (width 0.2) (layer "B.Cu") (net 4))
 (segment (start 159.41525 121.31525) (end 161.925 123.825) (width 0.2) (layer "B.Cu") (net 4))
 (segment (start 161.925 133.35) (end 197.64375 133.35) (width 0.2) (layer "B.Cu") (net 4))
 (segment (start 147.065 121.12625) (end 147.32 121.12625) (width 0.2) (layer "B.Cu") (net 4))
 (segment (start 178.435 83.185) (end 178.09 83.185) (width 0.2) (layer "B.Cu") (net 4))
 (segment (start 161.925 123.825) (end 161.925 133.35) (width 0.2) (layer "B.Cu") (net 4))
 (segment (start 147.32 121.12625) (end 147.6375 121.44375) (width 0.2) (layer "B.Cu") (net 4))
 (segment (start 147.6375 121.44375) (end 147.766 121.31525) (width 0.2) (layer "B.Cu") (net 4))
 (segment (start 200.025 104.775) (end 178.435 83.185) (width 0.2) (layer "B.Cu") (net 4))
 (segment (start 162.905 90.805) (end 163.2 91.1) (width 0.2) (layer "F.Cu") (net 11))
 (via (at 161.925 91.0875) (size 0.6) (drill 0.3) (layers "F.Cu" "B.Cu") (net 11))
 (segment (start 166.115 121.12625) (end 166.37 121.12625) (width 0.2) (layer "B.Cu") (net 11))
 (segment (start 161.324 116.08025) (end 161.324 91.0885) (width 0.2) (layer "B.Cu") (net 11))
 (segment (start 161.324 91.0885) (end 161.524 90.8885) (width 0.2) (layer "B.Cu") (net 11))
 (segment (start 166.37 121.12625) (end 161.324 116.08025) (width 0.2) (layer "B.Cu") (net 11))
 (segment (start 161.524 90.8885) (end 161.925 90.8885) (width 0.2) (layer "B.Cu") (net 11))
 (segment (start 161.925 90.8885) (end 161.925 91.0875) (width 0.2) (layer "B.Cu") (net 11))
 (segment (start 159.54375 90.4875) (end 161.76625 88.265) (width 0.2) (layer "F.Cu") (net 10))
 (segment (start 161.76625 88.265) (end 161.925 88.265) (width 0.2) (layer "F.Cu") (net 10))
 (segment (start 159.54375 92.86875) (end 159.54375 90.4875) (width 0.2) (layer "F.Cu") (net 10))
 (segment (start 161.925 95.25) (end 159.54375 92.86875) (width 0.2) (layer "F.Cu") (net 10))
 (via (at 161.925 95.25) (size 0.6) (drill 0.3) (layers "F.Cu" "B.Cu") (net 10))
 (segment (start 185.7375 121.44375) (end 183.427684 121.44375) (width 0.2) (layer "B.Cu") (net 10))
 (segment (start 183.427684 121.44375) (end 161.925 99.941066) (width 0.2) (layer "B.Cu") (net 10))
 (segment (start 161.925 99.941066) (end 161.925 95.25) (width 0.2) (layer "B.Cu") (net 10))
 (segment (start 185.165 121.12625) (end 185.42 121.12625) (width 0.2) (layer "B.Cu") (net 10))
 (segment (start 185.42 121.12625) (end 185.7375 121.44375) (width 0.2) (layer "B.Cu") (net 10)))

